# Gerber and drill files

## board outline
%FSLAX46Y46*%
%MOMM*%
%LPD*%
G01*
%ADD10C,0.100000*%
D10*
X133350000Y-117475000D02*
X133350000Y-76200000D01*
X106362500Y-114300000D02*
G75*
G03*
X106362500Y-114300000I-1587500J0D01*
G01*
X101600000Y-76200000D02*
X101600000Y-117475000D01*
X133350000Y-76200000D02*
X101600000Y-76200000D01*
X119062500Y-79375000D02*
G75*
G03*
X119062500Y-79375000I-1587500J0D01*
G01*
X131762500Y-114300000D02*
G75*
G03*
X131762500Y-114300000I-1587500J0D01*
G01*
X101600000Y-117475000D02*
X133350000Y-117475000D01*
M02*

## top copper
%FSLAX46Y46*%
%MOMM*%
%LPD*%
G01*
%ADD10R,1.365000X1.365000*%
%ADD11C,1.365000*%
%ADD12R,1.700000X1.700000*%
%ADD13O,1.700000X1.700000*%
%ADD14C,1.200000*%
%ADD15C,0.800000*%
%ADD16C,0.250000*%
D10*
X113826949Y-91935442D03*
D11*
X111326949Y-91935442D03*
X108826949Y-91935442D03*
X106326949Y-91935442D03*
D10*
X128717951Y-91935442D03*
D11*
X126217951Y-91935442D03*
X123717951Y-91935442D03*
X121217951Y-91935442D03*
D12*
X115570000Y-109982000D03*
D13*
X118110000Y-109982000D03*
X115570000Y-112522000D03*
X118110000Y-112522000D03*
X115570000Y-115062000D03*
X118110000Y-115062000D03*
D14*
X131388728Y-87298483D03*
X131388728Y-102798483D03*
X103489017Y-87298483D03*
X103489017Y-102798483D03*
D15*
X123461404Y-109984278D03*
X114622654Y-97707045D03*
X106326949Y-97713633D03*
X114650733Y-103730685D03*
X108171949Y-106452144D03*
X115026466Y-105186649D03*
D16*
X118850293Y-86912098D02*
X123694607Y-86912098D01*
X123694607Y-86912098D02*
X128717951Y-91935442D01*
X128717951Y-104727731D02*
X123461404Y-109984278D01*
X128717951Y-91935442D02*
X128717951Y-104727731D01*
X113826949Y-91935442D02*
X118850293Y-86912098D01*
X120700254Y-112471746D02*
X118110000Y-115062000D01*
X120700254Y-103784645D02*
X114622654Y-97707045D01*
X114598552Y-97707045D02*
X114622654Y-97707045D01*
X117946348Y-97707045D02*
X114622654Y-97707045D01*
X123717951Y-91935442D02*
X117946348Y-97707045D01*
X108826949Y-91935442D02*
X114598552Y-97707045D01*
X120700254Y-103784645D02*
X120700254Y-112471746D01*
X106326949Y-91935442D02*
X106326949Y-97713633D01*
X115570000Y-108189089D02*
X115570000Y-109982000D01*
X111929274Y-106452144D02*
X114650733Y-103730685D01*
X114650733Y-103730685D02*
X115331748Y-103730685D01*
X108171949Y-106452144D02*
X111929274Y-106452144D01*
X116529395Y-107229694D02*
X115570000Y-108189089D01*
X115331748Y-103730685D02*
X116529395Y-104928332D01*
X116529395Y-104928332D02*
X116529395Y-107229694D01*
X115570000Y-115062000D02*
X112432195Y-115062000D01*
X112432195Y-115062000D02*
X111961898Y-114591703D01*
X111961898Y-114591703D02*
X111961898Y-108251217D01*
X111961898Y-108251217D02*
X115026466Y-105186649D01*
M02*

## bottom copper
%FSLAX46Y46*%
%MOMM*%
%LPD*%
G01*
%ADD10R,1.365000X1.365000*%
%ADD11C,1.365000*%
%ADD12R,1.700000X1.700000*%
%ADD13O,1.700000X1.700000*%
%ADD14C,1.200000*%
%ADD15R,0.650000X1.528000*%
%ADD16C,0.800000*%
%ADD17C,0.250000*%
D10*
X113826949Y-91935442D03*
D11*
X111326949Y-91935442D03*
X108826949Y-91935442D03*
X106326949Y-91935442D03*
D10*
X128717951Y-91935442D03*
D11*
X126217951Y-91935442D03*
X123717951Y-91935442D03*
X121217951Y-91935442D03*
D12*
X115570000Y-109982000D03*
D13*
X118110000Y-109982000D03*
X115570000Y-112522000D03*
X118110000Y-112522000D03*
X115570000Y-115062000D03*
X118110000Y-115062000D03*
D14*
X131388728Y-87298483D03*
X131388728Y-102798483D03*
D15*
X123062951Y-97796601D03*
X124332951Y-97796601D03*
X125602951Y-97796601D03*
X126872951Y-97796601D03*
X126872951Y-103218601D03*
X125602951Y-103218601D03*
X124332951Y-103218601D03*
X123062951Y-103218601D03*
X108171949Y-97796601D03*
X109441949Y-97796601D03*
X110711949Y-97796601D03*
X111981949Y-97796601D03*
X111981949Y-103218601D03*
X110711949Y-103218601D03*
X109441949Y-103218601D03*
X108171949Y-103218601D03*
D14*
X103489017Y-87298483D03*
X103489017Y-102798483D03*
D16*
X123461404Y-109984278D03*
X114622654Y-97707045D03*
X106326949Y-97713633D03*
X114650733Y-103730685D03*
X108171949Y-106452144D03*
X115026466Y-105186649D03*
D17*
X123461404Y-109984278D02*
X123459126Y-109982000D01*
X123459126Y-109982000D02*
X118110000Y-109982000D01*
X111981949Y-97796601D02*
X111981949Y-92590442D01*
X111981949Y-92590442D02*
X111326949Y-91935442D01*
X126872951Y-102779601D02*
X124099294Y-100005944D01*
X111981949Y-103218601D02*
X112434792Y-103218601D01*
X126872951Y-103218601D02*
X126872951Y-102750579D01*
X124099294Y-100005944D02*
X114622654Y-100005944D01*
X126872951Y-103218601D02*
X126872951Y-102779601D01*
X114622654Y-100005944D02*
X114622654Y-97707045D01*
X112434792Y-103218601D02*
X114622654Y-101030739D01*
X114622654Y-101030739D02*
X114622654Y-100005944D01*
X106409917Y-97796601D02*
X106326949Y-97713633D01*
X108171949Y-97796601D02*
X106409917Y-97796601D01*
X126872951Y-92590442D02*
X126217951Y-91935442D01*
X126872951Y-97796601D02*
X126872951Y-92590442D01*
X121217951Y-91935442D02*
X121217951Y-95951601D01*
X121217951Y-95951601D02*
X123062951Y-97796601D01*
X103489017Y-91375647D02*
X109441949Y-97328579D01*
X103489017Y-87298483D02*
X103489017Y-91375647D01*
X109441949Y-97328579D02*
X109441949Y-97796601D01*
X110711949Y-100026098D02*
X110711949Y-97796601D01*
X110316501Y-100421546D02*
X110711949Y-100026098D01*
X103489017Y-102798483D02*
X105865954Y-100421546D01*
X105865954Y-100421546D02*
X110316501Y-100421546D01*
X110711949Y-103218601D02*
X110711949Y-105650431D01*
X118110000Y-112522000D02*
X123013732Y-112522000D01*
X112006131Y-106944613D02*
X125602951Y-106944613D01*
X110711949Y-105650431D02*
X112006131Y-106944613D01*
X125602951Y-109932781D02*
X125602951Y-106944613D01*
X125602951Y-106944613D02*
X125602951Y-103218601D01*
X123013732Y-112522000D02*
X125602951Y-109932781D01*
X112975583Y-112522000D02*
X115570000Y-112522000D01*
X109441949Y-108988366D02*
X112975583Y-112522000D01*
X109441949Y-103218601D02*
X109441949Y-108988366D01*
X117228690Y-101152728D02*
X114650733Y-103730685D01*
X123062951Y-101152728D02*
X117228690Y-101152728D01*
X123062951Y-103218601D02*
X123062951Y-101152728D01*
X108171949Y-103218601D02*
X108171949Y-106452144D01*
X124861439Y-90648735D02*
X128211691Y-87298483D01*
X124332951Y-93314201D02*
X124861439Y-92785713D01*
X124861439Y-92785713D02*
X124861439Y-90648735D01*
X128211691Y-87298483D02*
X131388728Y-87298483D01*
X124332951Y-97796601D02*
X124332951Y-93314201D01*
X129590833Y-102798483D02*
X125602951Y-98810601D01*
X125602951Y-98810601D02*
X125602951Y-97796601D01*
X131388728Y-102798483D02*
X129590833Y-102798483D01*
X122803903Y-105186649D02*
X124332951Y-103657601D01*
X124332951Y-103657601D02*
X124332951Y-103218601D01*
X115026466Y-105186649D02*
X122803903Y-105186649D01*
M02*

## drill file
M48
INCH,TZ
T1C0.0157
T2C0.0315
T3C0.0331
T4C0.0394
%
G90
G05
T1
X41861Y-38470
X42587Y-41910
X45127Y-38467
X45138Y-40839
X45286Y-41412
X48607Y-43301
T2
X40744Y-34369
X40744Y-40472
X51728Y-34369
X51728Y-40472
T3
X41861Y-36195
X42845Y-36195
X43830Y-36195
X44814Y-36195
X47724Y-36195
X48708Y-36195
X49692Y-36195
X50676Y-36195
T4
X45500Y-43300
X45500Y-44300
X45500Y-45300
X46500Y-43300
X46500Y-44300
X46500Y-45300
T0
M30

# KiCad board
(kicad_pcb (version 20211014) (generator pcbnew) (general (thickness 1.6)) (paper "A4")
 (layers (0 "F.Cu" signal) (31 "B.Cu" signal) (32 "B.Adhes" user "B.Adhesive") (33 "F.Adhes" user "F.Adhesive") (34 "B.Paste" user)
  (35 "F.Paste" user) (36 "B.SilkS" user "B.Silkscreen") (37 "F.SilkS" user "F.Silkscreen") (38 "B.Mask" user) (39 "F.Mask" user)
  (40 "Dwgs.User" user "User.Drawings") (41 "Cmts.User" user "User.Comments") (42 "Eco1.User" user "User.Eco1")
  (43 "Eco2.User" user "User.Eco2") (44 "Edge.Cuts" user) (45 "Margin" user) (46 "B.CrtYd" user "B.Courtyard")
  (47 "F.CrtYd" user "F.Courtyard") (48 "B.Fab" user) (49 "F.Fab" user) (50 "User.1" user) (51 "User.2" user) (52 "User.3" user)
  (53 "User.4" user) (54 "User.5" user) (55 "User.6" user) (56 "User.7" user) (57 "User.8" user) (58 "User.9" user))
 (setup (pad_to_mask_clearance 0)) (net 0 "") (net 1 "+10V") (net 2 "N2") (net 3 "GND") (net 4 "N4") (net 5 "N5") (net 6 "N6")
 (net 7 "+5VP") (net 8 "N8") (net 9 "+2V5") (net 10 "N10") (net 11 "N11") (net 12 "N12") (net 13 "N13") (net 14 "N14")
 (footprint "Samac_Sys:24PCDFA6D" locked (layer "F.Cu") (at 113.826949 91.935442)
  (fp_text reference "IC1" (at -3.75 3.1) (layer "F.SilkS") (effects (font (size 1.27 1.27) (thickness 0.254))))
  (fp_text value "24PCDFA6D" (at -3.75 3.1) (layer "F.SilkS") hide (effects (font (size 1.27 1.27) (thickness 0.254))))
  (pad "1" thru_hole rect locked (at 0 0) (size 1.365 1.365) (drill 0.84) (layers *.Cu *.Mask) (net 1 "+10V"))
  (pad "2" thru_hole circle locked (at -2.5 0) (size 1.365 1.365) (drill 0.84) (layers *.Cu *.Mask) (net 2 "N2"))
  (pad "3" thru_hole circle locked (at -5 0) (size 1.365 1.365) (drill 0.84) (layers *.Cu *.Mask) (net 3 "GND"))
  (pad "4" thru_hole circle locked (at -7.5 0) (size 1.365 1.365) (drill 0.84) (layers *.Cu *.Mask) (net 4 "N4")))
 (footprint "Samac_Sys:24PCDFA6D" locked (layer "F.Cu") (at 128.717951 91.935442)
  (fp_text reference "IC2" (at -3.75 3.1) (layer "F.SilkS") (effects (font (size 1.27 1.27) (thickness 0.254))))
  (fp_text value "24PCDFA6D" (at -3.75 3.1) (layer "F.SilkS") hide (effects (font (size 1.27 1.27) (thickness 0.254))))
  (pad "1" thru_hole rect locked (at 0 0) (size 1.365 1.365) (drill 0.84) (layers *.Cu *.Mask) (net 1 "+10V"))
  (pad "2" thru_hole circle locked (at -2.5 0) (size 1.365 1.365) (drill 0.84) (layers *.Cu *.Mask) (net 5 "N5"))
  (pad "3" thru_hole circle locked (at -5 0) (size 1.365 1.365) (drill 0.84) (layers *.Cu *.Mask) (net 3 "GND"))
  (pad "4" thru_hole circle locked (at -7.5 0) (size 1.365 1.365) (drill 0.84) (layers *.Cu *.Mask) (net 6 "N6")))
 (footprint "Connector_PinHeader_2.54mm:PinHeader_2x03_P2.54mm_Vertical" (layer "F.Cu") (at 115.57 109.982)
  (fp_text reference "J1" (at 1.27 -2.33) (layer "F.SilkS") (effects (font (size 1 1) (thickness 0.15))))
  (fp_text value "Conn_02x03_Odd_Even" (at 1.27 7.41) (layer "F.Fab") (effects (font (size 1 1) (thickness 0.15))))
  (pad "1" thru_hole rect locked (at 0 0) (size 1.7 1.7) (drill 1) (layers *.Cu *.Mask) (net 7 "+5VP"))
  (pad "2" thru_hole oval locked (at 2.54 0) (size 1.7 1.7) (drill 1) (layers *.Cu *.Mask) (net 1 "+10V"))
  (pad "3" thru_hole oval locked (at 0 2.54) (size 1.7 1.7) (drill 1) (layers *.Cu *.Mask) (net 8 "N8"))
  (pad "4" thru_hole oval locked (at 2.54 2.54) (size 1.7 1.7) (drill 1) (layers *.Cu *.Mask) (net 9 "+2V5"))
  (pad "5" thru_hole oval locked (at 0 5.08) (size 1.7 1.7) (drill 1) (layers *.Cu *.Mask) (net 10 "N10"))
  (pad "6" thru_hole oval locked (at 2.54 5.08) (size 1.7 1.7) (drill 1) (layers *.Cu *.Mask) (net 3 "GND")))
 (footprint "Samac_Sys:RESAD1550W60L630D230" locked (layer "B.Cu") (at 131.388728 87.298483 -90)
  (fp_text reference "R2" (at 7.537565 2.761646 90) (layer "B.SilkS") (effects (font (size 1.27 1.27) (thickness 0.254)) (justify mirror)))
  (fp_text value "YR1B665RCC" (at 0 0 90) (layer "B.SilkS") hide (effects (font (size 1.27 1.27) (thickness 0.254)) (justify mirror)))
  (pad "1" thru_hole circle locked (at 0 0 270) (size 1.2 1.2) (drill 0.8) (layers *.Cu *.Mask) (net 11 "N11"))
  (pad "2" thru_hole circle locked (at 15.5 0 270) (size 1.2 1.2) (drill 0.8) (layers *.Cu *.Mask) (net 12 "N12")))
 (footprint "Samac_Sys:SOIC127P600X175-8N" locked (layer "B.Cu") (at 124.967951 100.507601 -90)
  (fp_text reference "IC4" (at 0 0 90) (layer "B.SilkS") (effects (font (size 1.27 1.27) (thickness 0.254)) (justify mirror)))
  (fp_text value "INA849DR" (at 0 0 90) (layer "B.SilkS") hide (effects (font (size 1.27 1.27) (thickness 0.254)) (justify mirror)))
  (pad "1" smd rect locked (at -2.711 1.905 180) (size 0.65 1.528) (layers "B.Cu" "B.Paste" "B.Mask") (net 6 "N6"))
  (pad "2" smd rect locked (at -2.711 0.635 180) (size 0.65 1.528) (layers "B.Cu" "B.Paste" "B.Mask") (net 11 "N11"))
  (pad "3" smd rect locked (at -2.711 -0.635 180) (size 0.65 1.528) (layers "B.Cu" "B.Paste" "B.Mask") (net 12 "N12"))
  (pad "4" smd rect locked (at -2.711 -1.905 180) (size 0.65 1.528) (layers "B.Cu" "B.Paste" "B.Mask") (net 5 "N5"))
  (pad "5" smd rect locked (at 2.711 -1.905 180) (size 0.65 1.528) (layers "B.Cu" "B.Paste" "B.Mask") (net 3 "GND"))
  (pad "6" smd rect locked (at 2.711 -0.635 180) (size 0.65 1.528) (layers "B.Cu" "B.Paste" "B.Mask") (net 9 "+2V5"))
  (pad "7" smd rect locked (at 2.711 0.635 180) (size 0.65 1.528) (layers "B.Cu" "B.Paste" "B.Mask") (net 10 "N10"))
  (pad "8" smd rect locked (at 2.711 1.905 180) (size 0.65 1.528) (layers "B.Cu" "B.Paste" "B.Mask") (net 7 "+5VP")))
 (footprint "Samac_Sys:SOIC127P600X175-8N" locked (layer "B.Cu") (at 110.076949 100.507601 -90)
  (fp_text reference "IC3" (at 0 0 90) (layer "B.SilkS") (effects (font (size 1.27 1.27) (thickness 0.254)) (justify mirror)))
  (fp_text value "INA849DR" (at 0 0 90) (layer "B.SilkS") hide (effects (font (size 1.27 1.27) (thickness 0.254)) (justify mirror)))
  (pad "1" smd rect locked (at -2.711 1.905 180) (size 0.65 1.528) (layers "B.Cu" "B.Paste" "B.Mask") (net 4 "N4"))
  (pad "2" smd rect locked (at -2.711 0.635 180) (size 0.65 1.528) (layers "B.Cu" "B.Paste" "B.Mask") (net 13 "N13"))
  (pad "3" smd rect locked (at -2.711 -0.635 180) (size 0.65 1.528) (layers "B.Cu" "B.Paste" "B.Mask") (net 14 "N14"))
  (pad "4" smd rect locked (at -2.711 -1.905 180) (size 0.65 1.528) (layers "B.Cu" "B.Paste" "B.Mask") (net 2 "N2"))
  (pad "5" smd rect locked (at 2.711 -1.905 180) (size 0.65 1.528) (layers "B.Cu" "B.Paste" "B.Mask") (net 3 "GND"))
  (pad "6" smd rect locked (at 2.711 -0.635 180) (size 0.65 1.528) (layers "B.Cu" "B.Paste" "B.Mask") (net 9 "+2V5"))
  (pad "7" smd rect locked (at 2.711 0.635 180) (size 0.65 1.528) (layers "B.Cu" "B.Paste" "B.Mask") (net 8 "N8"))
  (pad "8" smd rect locked (at 2.711 1.905 180) (size 0.65 1.528) (layers "B.Cu" "B.Paste" "B.Mask") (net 7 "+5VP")))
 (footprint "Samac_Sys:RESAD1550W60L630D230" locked (layer "B.Cu") (at 103.489017 87.298483 -90)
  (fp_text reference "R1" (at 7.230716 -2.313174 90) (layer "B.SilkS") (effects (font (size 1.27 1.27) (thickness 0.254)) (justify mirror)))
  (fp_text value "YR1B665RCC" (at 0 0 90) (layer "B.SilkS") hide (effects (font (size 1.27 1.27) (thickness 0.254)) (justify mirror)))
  (pad "1" thru_hole circle locked (at 0 0 270) (size 1.2 1.2) (drill 0.8) (layers *.Cu *.Mask) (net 13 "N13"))
  (pad "2" thru_hole circle locked (at 15.5 0 270) (size 1.2 1.2) (drill 0.8) (layers *.Cu *.Mask) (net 14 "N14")))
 (gr_line (start 133.35 117.475) (end 133.35 76.2) (layer "Edge.Cuts") (width 0.1))
 (gr_circle (center 104.775 114.3) (end 106.3625 114.3) (layer "Edge.Cuts") (width 0.1) (fill none))
 (gr_circle (center 117.475 79.375) (end 119.0625 79.375) (layer "Edge.Cuts") (width 0.1) (fill none))
 (gr_line (start 101.6 76.2) (end 101.6 117.475) (layer "Edge.Cuts") (width 0.1))
 (gr_line (start 133.35 76.2) (end 101.6 76.2) (layer "Edge.Cuts") (width 0.1))
 (gr_circle (center 130.175 114.3) (end 131.7625 114.3) (layer "Edge.Cuts") (width 0.1) (fill none))
 (gr_line (start 101.6 117.475) (end 133.35 117.475) (layer "Edge.Cuts") (width 0.1))
 (segment (start 118.850293 86.912098) (end 123.694607 86.912098) (width 0.25) (layer "F.Cu") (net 1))
 (segment (start 123.694607 86.912098) (end 128.717951 91.935442) (width 0.25) (layer "F.Cu") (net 1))
 (segment (start 128.717951 104.727731) (end 123.461404 109.984278) (width 0.25) (layer "F.Cu") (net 1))
 (segment (start 128.717951 91.935442) (end 128.717951 104.727731) (width 0.25) (layer "F.Cu") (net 1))
 (segment (start 113.826949 91.935442) (end 118.850293 86.912098) (width 0.25) (layer "F.Cu") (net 1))
 (via (at 123.461404 109.984278) (size 0.8) (drill 0.4) (layers "F.Cu" "B.Cu") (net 1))
 (segment (start 123.461404 109.984278) (end 123.459126 109.982) (width 0.25) (layer "B.Cu") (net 1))
 (segment (start 123.459126 109.982) (end 118.11 109.982) (width 0.25) (layer "B.Cu") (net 1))
 (segment (start 111.981949 97.796601) (end 111.981949 92.590442) (width 0.25) (layer "B.Cu") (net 2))
 (segment (start 111.981949 92.590442) (end 111.326949 91.935442) (width 0.25) (layer "B.Cu") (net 2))
 (segment (start 120.700254 112.471746) (end 118.11 115.062) (width 0.25) (layer "F.Cu") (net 3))
 (segment (start 120.700254 103.784645) (end 114.622654 97.707045) (width 0.25) (layer "F.Cu") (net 3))
 (segment (start 114.598552 97.707045) (end 114.622654 97.707045) (width 0.25) (layer "F.Cu") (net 3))
 (segment (start 117.946348 97.707045) (end 114.622654 97.707045) (width 0.25) (layer "F.Cu") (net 3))
 (segment (start 123.717951 91.935442) (end 117.946348 97.707045) (width 0.25) (layer "F.Cu") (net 3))
 (segment (start 108.826949 91.935442) (end 114.598552 97.707045) (width 0.25) (layer "F.Cu") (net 3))
 (segment (start 120.700254 103.784645) (end 120.700254 112.471746) (width 0.25) (layer "F.Cu") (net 3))
 (via (at 114.622654 97.707045) (size 0.8) (drill 0.4) (layers "F.Cu" "B.Cu") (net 3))
 (segment (start 126.872951 102.779601) (end 124.099294 100.005944) (width 0.25) (layer "B.Cu") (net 3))
 (segment (start 111.981949 103.218601) (end 112.434792 103.218601) (width 0.25) (layer "B.Cu") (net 3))
 (segment (start 126.872951 103.218601) (end 126.872951 102.750579) (width 0.25) (layer "B.Cu") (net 3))
 (segment (start 124.099294 100.005944) (end 114.622654 100.005944) (width 0.25) (layer "B.Cu") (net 3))
 (segment (start 126.872951 103.218601) (end 126.872951 102.779601) (width 0.25) (layer "B.Cu") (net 3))
 (segment (start 114.622654 100.005944) (end 114.622654 97.707045) (width 0.25) (layer "B.Cu") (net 3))
 (segment (start 112.434792 103.218601) (end 114.622654 101.030739) (width 0.25) (layer "B.Cu") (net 3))
 (segment (start 114.622654 101.030739) (end 114.622654 100.005944) (width 0.25) (layer "B.Cu") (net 3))
 (segment (start 106.326949 91.935442) (end 106.326949 97.713633) (width 0.25) (layer "F.Cu") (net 4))
 (via (at 106.326949 97.713633) (size 0.8) (drill 0.4) (layers "F.Cu" "B.Cu") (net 4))
 (segment (start 106.409917 97.796601) (end 106.326949 97.713633) (width 0.25) (layer "B.Cu") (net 4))
 (segment (start 108.171949 97.796601) (end 106.409917 97.796601) (width 0.25) (layer "B.Cu") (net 4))
 (segment (start 126.872951 92.590442) (end 126.217951 91.935442) (width 0.25) (layer "B.Cu") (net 5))
 (segment (start 126.872951 97.796601) (end 126.872951 92.590442) (width 0.25) (layer "B.Cu") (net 5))
 (segment (start 121.217951 91.935442) (end 121.217951 95.951601) (width 0.25) (layer "B.Cu") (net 6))
 (segment (start 121.217951 95.951601) (end 123.062951 97.796601) (width 0.25) (layer "B.Cu") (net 6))
 (segment (start 103.489017 91.375647) (end 109.441949 97.328579) (width 0.25) (layer "B.Cu") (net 13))
 (segment (start 103.489017 87.298483) (end 103.489017 91.375647) (width 0.25) (layer "B.Cu") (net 13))
 (segment (start 109.441949 97.328579) (end 109.441949 97.796601) (width 0.25) (layer "B.Cu") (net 13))
 (segment (start 110.711949 100.026098) (end 110.711949 97.796601) (width 0.25) (layer "B.Cu") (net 14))
 (segment (start 110.316501 100.421546) (end 110.711949 100.026098) (width 0.25) (layer "B.Cu") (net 14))
 (segment (start 103.489017 102.798483) (end 105.865954 100.421546) (width 0.25) (layer "B.Cu") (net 14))
 (segment (start 105.865954 100.421546) (end 110.316501 100.421546) (width 0.25) (layer "B.Cu") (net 14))
 (segment (start 110.711949 103.218601) (end 110.711949 105.650431) (width 0.25) (layer "B.Cu") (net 9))
 (segment (start 118.11 112.522) (end 123.013732 112.522) (width 0.25) (layer "B.Cu") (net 9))
 (segment (start 112.006131 106.944613) (end 125.602951 106.944613) (width 0.25) (layer "B.Cu") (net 9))
 (segment (start 110.711949 105.650431) (end 112.006131 106.944613) (width 0.25) (layer "B.Cu") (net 9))
 (segment (start 125.602951 109.932781) (end 125.602951 106.944613) (width 0.25) (layer "B.Cu") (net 9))
 (segment (start 125.602951 106.944613) (end 125.602951 103.218601) (width 0.25) (layer "B.Cu") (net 9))
 (segment (start 123.013732 112.522) (end 125.602951 109.932781) (width 0.25) (layer "B.Cu") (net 9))
 (segment (start 112.975583 112.522) (end 115.57 112.522) (width 0.25) (layer "B.Cu") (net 8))
 (segment (start 109.441949 108.988366) (end 112.975583 112.522) (width 0.25) (layer "B.Cu") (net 8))
 (segment (start 109.441949 103.218601) (end 109.441949 108.988366) (width 0.25) (layer "B.Cu") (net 8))
 (segment (start 115.57 108.189089) (end 115.57 109.982) (width 0.25) (layer "F.Cu") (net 7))
 (segment (start 111.929274 106.452144) (end 114.650733 103.730685) (width 0.25) (layer "F.Cu") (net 7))
 (segment (start 114.650733 103.730685) (end 115.331748 103.730685) (width 0.25) (layer "F.Cu") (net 7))
 (segment (start 108.171949 106.452144) (end 111.929274 106.452144) (width 0.25) (layer "F.Cu") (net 7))
 (segment (start 116.529395 107.229694) (end 115.57 108.189089) (width 0.25) (layer "F.Cu") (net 7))
 (segment (start 115.331748 103.730685) (end 116.529395 104.928332) (width 0.25) (layer "F.Cu") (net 7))
 (segment (start 116.529395 104.928332) (end 116.529395 107.229694) (width 0.25) (layer "F.Cu") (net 7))
 (via (at 114.650733 103.730685) (size 0.8) (drill 0.4) (layers "F.Cu" "B.Cu") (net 7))
 (via (at 108.171949 106.452144) (size 0.8) (drill 0.4) (layers "F.Cu" "B.Cu") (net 7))
 (segment (start 117.22869 101.152728) (end 114.650733 103.730685) (width 0.25) (layer "B.Cu") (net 7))
 (segment (start 123.062951 101.152728) (end 117.22869 101.152728) (width 0.25) (layer "B.Cu") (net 7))
 (segment (start 123.062951 103.218601) (end 123.062951 101.152728) (width 0.25) (layer "B.Cu") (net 7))
 (segment (start 108.171949 103.218601) (end 108.171949 106.452144) (width 0.25) (layer "B.Cu") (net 7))
 (segment (start 124.861439 90.648735) (end 128.211691 87.298483) (width 0.25) (layer "B.Cu") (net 11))
 (segment (start 124.332951 93.314201) (end 124.861439 92.785713) (width 0.25) (layer "B.Cu") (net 11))
 (segment (start 124.861439 92.785713) (end 124.861439 90.648735) (width 0.25) (layer "B.Cu") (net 11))
 (segment (start 128.211691 87.298483) (end 131.388728 87.298483) (width 0.25) (layer "B.Cu") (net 11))
 (segment (start 124.332951 97.796601) (end 124.332951 93.314201) (width 0.25) (layer "B.Cu") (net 11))
 (segment (start 129.590833 102.798483) (end 125.602951 98.810601) (width 0.25) (layer "B.Cu") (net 12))
 (segment (start 125.602951 98.810601) (end 125.602951 97.796601) (width 0.25) (layer "B.Cu") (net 12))
 (segment (start 131.388728 102.798483) (end 129.590833 102.798483) (width 0.25) (layer "B.Cu") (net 12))
 (segment (start 115.57 115.062) (end 112.432195 115.062) (width 0.25) (layer "F.Cu") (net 10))
 (segment (start 112.432195 115.062) (end 111.961898 114.591703) (width 0.25) (layer "F.Cu") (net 10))
 (segment (start 111.961898 114.591703) (end 111.961898 108.251217) (width 0.25) (layer "F.Cu") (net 10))
 (segment (start 111.961898 108.251217) (end 115.026466 105.186649) (width 0.25) (layer "F.Cu") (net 10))
 (via (at 115.026466 105.186649) (size 0.8) (drill 0.4) (layers "F.Cu" "B.Cu") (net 10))
 (segment (start 122.803903 105.186649) (end 124.332951 103.657601) (width 0.25) (layer "B.Cu") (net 10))
 (segment (start 124.332951 103.657601) (end 124.332951 103.218601) (width 0.25) (layer "B.Cu") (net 10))
 (segment (start 115.026466 105.186649) (end 122.803903 105.186649) (width 0.25) (layer "B.Cu") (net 10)))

